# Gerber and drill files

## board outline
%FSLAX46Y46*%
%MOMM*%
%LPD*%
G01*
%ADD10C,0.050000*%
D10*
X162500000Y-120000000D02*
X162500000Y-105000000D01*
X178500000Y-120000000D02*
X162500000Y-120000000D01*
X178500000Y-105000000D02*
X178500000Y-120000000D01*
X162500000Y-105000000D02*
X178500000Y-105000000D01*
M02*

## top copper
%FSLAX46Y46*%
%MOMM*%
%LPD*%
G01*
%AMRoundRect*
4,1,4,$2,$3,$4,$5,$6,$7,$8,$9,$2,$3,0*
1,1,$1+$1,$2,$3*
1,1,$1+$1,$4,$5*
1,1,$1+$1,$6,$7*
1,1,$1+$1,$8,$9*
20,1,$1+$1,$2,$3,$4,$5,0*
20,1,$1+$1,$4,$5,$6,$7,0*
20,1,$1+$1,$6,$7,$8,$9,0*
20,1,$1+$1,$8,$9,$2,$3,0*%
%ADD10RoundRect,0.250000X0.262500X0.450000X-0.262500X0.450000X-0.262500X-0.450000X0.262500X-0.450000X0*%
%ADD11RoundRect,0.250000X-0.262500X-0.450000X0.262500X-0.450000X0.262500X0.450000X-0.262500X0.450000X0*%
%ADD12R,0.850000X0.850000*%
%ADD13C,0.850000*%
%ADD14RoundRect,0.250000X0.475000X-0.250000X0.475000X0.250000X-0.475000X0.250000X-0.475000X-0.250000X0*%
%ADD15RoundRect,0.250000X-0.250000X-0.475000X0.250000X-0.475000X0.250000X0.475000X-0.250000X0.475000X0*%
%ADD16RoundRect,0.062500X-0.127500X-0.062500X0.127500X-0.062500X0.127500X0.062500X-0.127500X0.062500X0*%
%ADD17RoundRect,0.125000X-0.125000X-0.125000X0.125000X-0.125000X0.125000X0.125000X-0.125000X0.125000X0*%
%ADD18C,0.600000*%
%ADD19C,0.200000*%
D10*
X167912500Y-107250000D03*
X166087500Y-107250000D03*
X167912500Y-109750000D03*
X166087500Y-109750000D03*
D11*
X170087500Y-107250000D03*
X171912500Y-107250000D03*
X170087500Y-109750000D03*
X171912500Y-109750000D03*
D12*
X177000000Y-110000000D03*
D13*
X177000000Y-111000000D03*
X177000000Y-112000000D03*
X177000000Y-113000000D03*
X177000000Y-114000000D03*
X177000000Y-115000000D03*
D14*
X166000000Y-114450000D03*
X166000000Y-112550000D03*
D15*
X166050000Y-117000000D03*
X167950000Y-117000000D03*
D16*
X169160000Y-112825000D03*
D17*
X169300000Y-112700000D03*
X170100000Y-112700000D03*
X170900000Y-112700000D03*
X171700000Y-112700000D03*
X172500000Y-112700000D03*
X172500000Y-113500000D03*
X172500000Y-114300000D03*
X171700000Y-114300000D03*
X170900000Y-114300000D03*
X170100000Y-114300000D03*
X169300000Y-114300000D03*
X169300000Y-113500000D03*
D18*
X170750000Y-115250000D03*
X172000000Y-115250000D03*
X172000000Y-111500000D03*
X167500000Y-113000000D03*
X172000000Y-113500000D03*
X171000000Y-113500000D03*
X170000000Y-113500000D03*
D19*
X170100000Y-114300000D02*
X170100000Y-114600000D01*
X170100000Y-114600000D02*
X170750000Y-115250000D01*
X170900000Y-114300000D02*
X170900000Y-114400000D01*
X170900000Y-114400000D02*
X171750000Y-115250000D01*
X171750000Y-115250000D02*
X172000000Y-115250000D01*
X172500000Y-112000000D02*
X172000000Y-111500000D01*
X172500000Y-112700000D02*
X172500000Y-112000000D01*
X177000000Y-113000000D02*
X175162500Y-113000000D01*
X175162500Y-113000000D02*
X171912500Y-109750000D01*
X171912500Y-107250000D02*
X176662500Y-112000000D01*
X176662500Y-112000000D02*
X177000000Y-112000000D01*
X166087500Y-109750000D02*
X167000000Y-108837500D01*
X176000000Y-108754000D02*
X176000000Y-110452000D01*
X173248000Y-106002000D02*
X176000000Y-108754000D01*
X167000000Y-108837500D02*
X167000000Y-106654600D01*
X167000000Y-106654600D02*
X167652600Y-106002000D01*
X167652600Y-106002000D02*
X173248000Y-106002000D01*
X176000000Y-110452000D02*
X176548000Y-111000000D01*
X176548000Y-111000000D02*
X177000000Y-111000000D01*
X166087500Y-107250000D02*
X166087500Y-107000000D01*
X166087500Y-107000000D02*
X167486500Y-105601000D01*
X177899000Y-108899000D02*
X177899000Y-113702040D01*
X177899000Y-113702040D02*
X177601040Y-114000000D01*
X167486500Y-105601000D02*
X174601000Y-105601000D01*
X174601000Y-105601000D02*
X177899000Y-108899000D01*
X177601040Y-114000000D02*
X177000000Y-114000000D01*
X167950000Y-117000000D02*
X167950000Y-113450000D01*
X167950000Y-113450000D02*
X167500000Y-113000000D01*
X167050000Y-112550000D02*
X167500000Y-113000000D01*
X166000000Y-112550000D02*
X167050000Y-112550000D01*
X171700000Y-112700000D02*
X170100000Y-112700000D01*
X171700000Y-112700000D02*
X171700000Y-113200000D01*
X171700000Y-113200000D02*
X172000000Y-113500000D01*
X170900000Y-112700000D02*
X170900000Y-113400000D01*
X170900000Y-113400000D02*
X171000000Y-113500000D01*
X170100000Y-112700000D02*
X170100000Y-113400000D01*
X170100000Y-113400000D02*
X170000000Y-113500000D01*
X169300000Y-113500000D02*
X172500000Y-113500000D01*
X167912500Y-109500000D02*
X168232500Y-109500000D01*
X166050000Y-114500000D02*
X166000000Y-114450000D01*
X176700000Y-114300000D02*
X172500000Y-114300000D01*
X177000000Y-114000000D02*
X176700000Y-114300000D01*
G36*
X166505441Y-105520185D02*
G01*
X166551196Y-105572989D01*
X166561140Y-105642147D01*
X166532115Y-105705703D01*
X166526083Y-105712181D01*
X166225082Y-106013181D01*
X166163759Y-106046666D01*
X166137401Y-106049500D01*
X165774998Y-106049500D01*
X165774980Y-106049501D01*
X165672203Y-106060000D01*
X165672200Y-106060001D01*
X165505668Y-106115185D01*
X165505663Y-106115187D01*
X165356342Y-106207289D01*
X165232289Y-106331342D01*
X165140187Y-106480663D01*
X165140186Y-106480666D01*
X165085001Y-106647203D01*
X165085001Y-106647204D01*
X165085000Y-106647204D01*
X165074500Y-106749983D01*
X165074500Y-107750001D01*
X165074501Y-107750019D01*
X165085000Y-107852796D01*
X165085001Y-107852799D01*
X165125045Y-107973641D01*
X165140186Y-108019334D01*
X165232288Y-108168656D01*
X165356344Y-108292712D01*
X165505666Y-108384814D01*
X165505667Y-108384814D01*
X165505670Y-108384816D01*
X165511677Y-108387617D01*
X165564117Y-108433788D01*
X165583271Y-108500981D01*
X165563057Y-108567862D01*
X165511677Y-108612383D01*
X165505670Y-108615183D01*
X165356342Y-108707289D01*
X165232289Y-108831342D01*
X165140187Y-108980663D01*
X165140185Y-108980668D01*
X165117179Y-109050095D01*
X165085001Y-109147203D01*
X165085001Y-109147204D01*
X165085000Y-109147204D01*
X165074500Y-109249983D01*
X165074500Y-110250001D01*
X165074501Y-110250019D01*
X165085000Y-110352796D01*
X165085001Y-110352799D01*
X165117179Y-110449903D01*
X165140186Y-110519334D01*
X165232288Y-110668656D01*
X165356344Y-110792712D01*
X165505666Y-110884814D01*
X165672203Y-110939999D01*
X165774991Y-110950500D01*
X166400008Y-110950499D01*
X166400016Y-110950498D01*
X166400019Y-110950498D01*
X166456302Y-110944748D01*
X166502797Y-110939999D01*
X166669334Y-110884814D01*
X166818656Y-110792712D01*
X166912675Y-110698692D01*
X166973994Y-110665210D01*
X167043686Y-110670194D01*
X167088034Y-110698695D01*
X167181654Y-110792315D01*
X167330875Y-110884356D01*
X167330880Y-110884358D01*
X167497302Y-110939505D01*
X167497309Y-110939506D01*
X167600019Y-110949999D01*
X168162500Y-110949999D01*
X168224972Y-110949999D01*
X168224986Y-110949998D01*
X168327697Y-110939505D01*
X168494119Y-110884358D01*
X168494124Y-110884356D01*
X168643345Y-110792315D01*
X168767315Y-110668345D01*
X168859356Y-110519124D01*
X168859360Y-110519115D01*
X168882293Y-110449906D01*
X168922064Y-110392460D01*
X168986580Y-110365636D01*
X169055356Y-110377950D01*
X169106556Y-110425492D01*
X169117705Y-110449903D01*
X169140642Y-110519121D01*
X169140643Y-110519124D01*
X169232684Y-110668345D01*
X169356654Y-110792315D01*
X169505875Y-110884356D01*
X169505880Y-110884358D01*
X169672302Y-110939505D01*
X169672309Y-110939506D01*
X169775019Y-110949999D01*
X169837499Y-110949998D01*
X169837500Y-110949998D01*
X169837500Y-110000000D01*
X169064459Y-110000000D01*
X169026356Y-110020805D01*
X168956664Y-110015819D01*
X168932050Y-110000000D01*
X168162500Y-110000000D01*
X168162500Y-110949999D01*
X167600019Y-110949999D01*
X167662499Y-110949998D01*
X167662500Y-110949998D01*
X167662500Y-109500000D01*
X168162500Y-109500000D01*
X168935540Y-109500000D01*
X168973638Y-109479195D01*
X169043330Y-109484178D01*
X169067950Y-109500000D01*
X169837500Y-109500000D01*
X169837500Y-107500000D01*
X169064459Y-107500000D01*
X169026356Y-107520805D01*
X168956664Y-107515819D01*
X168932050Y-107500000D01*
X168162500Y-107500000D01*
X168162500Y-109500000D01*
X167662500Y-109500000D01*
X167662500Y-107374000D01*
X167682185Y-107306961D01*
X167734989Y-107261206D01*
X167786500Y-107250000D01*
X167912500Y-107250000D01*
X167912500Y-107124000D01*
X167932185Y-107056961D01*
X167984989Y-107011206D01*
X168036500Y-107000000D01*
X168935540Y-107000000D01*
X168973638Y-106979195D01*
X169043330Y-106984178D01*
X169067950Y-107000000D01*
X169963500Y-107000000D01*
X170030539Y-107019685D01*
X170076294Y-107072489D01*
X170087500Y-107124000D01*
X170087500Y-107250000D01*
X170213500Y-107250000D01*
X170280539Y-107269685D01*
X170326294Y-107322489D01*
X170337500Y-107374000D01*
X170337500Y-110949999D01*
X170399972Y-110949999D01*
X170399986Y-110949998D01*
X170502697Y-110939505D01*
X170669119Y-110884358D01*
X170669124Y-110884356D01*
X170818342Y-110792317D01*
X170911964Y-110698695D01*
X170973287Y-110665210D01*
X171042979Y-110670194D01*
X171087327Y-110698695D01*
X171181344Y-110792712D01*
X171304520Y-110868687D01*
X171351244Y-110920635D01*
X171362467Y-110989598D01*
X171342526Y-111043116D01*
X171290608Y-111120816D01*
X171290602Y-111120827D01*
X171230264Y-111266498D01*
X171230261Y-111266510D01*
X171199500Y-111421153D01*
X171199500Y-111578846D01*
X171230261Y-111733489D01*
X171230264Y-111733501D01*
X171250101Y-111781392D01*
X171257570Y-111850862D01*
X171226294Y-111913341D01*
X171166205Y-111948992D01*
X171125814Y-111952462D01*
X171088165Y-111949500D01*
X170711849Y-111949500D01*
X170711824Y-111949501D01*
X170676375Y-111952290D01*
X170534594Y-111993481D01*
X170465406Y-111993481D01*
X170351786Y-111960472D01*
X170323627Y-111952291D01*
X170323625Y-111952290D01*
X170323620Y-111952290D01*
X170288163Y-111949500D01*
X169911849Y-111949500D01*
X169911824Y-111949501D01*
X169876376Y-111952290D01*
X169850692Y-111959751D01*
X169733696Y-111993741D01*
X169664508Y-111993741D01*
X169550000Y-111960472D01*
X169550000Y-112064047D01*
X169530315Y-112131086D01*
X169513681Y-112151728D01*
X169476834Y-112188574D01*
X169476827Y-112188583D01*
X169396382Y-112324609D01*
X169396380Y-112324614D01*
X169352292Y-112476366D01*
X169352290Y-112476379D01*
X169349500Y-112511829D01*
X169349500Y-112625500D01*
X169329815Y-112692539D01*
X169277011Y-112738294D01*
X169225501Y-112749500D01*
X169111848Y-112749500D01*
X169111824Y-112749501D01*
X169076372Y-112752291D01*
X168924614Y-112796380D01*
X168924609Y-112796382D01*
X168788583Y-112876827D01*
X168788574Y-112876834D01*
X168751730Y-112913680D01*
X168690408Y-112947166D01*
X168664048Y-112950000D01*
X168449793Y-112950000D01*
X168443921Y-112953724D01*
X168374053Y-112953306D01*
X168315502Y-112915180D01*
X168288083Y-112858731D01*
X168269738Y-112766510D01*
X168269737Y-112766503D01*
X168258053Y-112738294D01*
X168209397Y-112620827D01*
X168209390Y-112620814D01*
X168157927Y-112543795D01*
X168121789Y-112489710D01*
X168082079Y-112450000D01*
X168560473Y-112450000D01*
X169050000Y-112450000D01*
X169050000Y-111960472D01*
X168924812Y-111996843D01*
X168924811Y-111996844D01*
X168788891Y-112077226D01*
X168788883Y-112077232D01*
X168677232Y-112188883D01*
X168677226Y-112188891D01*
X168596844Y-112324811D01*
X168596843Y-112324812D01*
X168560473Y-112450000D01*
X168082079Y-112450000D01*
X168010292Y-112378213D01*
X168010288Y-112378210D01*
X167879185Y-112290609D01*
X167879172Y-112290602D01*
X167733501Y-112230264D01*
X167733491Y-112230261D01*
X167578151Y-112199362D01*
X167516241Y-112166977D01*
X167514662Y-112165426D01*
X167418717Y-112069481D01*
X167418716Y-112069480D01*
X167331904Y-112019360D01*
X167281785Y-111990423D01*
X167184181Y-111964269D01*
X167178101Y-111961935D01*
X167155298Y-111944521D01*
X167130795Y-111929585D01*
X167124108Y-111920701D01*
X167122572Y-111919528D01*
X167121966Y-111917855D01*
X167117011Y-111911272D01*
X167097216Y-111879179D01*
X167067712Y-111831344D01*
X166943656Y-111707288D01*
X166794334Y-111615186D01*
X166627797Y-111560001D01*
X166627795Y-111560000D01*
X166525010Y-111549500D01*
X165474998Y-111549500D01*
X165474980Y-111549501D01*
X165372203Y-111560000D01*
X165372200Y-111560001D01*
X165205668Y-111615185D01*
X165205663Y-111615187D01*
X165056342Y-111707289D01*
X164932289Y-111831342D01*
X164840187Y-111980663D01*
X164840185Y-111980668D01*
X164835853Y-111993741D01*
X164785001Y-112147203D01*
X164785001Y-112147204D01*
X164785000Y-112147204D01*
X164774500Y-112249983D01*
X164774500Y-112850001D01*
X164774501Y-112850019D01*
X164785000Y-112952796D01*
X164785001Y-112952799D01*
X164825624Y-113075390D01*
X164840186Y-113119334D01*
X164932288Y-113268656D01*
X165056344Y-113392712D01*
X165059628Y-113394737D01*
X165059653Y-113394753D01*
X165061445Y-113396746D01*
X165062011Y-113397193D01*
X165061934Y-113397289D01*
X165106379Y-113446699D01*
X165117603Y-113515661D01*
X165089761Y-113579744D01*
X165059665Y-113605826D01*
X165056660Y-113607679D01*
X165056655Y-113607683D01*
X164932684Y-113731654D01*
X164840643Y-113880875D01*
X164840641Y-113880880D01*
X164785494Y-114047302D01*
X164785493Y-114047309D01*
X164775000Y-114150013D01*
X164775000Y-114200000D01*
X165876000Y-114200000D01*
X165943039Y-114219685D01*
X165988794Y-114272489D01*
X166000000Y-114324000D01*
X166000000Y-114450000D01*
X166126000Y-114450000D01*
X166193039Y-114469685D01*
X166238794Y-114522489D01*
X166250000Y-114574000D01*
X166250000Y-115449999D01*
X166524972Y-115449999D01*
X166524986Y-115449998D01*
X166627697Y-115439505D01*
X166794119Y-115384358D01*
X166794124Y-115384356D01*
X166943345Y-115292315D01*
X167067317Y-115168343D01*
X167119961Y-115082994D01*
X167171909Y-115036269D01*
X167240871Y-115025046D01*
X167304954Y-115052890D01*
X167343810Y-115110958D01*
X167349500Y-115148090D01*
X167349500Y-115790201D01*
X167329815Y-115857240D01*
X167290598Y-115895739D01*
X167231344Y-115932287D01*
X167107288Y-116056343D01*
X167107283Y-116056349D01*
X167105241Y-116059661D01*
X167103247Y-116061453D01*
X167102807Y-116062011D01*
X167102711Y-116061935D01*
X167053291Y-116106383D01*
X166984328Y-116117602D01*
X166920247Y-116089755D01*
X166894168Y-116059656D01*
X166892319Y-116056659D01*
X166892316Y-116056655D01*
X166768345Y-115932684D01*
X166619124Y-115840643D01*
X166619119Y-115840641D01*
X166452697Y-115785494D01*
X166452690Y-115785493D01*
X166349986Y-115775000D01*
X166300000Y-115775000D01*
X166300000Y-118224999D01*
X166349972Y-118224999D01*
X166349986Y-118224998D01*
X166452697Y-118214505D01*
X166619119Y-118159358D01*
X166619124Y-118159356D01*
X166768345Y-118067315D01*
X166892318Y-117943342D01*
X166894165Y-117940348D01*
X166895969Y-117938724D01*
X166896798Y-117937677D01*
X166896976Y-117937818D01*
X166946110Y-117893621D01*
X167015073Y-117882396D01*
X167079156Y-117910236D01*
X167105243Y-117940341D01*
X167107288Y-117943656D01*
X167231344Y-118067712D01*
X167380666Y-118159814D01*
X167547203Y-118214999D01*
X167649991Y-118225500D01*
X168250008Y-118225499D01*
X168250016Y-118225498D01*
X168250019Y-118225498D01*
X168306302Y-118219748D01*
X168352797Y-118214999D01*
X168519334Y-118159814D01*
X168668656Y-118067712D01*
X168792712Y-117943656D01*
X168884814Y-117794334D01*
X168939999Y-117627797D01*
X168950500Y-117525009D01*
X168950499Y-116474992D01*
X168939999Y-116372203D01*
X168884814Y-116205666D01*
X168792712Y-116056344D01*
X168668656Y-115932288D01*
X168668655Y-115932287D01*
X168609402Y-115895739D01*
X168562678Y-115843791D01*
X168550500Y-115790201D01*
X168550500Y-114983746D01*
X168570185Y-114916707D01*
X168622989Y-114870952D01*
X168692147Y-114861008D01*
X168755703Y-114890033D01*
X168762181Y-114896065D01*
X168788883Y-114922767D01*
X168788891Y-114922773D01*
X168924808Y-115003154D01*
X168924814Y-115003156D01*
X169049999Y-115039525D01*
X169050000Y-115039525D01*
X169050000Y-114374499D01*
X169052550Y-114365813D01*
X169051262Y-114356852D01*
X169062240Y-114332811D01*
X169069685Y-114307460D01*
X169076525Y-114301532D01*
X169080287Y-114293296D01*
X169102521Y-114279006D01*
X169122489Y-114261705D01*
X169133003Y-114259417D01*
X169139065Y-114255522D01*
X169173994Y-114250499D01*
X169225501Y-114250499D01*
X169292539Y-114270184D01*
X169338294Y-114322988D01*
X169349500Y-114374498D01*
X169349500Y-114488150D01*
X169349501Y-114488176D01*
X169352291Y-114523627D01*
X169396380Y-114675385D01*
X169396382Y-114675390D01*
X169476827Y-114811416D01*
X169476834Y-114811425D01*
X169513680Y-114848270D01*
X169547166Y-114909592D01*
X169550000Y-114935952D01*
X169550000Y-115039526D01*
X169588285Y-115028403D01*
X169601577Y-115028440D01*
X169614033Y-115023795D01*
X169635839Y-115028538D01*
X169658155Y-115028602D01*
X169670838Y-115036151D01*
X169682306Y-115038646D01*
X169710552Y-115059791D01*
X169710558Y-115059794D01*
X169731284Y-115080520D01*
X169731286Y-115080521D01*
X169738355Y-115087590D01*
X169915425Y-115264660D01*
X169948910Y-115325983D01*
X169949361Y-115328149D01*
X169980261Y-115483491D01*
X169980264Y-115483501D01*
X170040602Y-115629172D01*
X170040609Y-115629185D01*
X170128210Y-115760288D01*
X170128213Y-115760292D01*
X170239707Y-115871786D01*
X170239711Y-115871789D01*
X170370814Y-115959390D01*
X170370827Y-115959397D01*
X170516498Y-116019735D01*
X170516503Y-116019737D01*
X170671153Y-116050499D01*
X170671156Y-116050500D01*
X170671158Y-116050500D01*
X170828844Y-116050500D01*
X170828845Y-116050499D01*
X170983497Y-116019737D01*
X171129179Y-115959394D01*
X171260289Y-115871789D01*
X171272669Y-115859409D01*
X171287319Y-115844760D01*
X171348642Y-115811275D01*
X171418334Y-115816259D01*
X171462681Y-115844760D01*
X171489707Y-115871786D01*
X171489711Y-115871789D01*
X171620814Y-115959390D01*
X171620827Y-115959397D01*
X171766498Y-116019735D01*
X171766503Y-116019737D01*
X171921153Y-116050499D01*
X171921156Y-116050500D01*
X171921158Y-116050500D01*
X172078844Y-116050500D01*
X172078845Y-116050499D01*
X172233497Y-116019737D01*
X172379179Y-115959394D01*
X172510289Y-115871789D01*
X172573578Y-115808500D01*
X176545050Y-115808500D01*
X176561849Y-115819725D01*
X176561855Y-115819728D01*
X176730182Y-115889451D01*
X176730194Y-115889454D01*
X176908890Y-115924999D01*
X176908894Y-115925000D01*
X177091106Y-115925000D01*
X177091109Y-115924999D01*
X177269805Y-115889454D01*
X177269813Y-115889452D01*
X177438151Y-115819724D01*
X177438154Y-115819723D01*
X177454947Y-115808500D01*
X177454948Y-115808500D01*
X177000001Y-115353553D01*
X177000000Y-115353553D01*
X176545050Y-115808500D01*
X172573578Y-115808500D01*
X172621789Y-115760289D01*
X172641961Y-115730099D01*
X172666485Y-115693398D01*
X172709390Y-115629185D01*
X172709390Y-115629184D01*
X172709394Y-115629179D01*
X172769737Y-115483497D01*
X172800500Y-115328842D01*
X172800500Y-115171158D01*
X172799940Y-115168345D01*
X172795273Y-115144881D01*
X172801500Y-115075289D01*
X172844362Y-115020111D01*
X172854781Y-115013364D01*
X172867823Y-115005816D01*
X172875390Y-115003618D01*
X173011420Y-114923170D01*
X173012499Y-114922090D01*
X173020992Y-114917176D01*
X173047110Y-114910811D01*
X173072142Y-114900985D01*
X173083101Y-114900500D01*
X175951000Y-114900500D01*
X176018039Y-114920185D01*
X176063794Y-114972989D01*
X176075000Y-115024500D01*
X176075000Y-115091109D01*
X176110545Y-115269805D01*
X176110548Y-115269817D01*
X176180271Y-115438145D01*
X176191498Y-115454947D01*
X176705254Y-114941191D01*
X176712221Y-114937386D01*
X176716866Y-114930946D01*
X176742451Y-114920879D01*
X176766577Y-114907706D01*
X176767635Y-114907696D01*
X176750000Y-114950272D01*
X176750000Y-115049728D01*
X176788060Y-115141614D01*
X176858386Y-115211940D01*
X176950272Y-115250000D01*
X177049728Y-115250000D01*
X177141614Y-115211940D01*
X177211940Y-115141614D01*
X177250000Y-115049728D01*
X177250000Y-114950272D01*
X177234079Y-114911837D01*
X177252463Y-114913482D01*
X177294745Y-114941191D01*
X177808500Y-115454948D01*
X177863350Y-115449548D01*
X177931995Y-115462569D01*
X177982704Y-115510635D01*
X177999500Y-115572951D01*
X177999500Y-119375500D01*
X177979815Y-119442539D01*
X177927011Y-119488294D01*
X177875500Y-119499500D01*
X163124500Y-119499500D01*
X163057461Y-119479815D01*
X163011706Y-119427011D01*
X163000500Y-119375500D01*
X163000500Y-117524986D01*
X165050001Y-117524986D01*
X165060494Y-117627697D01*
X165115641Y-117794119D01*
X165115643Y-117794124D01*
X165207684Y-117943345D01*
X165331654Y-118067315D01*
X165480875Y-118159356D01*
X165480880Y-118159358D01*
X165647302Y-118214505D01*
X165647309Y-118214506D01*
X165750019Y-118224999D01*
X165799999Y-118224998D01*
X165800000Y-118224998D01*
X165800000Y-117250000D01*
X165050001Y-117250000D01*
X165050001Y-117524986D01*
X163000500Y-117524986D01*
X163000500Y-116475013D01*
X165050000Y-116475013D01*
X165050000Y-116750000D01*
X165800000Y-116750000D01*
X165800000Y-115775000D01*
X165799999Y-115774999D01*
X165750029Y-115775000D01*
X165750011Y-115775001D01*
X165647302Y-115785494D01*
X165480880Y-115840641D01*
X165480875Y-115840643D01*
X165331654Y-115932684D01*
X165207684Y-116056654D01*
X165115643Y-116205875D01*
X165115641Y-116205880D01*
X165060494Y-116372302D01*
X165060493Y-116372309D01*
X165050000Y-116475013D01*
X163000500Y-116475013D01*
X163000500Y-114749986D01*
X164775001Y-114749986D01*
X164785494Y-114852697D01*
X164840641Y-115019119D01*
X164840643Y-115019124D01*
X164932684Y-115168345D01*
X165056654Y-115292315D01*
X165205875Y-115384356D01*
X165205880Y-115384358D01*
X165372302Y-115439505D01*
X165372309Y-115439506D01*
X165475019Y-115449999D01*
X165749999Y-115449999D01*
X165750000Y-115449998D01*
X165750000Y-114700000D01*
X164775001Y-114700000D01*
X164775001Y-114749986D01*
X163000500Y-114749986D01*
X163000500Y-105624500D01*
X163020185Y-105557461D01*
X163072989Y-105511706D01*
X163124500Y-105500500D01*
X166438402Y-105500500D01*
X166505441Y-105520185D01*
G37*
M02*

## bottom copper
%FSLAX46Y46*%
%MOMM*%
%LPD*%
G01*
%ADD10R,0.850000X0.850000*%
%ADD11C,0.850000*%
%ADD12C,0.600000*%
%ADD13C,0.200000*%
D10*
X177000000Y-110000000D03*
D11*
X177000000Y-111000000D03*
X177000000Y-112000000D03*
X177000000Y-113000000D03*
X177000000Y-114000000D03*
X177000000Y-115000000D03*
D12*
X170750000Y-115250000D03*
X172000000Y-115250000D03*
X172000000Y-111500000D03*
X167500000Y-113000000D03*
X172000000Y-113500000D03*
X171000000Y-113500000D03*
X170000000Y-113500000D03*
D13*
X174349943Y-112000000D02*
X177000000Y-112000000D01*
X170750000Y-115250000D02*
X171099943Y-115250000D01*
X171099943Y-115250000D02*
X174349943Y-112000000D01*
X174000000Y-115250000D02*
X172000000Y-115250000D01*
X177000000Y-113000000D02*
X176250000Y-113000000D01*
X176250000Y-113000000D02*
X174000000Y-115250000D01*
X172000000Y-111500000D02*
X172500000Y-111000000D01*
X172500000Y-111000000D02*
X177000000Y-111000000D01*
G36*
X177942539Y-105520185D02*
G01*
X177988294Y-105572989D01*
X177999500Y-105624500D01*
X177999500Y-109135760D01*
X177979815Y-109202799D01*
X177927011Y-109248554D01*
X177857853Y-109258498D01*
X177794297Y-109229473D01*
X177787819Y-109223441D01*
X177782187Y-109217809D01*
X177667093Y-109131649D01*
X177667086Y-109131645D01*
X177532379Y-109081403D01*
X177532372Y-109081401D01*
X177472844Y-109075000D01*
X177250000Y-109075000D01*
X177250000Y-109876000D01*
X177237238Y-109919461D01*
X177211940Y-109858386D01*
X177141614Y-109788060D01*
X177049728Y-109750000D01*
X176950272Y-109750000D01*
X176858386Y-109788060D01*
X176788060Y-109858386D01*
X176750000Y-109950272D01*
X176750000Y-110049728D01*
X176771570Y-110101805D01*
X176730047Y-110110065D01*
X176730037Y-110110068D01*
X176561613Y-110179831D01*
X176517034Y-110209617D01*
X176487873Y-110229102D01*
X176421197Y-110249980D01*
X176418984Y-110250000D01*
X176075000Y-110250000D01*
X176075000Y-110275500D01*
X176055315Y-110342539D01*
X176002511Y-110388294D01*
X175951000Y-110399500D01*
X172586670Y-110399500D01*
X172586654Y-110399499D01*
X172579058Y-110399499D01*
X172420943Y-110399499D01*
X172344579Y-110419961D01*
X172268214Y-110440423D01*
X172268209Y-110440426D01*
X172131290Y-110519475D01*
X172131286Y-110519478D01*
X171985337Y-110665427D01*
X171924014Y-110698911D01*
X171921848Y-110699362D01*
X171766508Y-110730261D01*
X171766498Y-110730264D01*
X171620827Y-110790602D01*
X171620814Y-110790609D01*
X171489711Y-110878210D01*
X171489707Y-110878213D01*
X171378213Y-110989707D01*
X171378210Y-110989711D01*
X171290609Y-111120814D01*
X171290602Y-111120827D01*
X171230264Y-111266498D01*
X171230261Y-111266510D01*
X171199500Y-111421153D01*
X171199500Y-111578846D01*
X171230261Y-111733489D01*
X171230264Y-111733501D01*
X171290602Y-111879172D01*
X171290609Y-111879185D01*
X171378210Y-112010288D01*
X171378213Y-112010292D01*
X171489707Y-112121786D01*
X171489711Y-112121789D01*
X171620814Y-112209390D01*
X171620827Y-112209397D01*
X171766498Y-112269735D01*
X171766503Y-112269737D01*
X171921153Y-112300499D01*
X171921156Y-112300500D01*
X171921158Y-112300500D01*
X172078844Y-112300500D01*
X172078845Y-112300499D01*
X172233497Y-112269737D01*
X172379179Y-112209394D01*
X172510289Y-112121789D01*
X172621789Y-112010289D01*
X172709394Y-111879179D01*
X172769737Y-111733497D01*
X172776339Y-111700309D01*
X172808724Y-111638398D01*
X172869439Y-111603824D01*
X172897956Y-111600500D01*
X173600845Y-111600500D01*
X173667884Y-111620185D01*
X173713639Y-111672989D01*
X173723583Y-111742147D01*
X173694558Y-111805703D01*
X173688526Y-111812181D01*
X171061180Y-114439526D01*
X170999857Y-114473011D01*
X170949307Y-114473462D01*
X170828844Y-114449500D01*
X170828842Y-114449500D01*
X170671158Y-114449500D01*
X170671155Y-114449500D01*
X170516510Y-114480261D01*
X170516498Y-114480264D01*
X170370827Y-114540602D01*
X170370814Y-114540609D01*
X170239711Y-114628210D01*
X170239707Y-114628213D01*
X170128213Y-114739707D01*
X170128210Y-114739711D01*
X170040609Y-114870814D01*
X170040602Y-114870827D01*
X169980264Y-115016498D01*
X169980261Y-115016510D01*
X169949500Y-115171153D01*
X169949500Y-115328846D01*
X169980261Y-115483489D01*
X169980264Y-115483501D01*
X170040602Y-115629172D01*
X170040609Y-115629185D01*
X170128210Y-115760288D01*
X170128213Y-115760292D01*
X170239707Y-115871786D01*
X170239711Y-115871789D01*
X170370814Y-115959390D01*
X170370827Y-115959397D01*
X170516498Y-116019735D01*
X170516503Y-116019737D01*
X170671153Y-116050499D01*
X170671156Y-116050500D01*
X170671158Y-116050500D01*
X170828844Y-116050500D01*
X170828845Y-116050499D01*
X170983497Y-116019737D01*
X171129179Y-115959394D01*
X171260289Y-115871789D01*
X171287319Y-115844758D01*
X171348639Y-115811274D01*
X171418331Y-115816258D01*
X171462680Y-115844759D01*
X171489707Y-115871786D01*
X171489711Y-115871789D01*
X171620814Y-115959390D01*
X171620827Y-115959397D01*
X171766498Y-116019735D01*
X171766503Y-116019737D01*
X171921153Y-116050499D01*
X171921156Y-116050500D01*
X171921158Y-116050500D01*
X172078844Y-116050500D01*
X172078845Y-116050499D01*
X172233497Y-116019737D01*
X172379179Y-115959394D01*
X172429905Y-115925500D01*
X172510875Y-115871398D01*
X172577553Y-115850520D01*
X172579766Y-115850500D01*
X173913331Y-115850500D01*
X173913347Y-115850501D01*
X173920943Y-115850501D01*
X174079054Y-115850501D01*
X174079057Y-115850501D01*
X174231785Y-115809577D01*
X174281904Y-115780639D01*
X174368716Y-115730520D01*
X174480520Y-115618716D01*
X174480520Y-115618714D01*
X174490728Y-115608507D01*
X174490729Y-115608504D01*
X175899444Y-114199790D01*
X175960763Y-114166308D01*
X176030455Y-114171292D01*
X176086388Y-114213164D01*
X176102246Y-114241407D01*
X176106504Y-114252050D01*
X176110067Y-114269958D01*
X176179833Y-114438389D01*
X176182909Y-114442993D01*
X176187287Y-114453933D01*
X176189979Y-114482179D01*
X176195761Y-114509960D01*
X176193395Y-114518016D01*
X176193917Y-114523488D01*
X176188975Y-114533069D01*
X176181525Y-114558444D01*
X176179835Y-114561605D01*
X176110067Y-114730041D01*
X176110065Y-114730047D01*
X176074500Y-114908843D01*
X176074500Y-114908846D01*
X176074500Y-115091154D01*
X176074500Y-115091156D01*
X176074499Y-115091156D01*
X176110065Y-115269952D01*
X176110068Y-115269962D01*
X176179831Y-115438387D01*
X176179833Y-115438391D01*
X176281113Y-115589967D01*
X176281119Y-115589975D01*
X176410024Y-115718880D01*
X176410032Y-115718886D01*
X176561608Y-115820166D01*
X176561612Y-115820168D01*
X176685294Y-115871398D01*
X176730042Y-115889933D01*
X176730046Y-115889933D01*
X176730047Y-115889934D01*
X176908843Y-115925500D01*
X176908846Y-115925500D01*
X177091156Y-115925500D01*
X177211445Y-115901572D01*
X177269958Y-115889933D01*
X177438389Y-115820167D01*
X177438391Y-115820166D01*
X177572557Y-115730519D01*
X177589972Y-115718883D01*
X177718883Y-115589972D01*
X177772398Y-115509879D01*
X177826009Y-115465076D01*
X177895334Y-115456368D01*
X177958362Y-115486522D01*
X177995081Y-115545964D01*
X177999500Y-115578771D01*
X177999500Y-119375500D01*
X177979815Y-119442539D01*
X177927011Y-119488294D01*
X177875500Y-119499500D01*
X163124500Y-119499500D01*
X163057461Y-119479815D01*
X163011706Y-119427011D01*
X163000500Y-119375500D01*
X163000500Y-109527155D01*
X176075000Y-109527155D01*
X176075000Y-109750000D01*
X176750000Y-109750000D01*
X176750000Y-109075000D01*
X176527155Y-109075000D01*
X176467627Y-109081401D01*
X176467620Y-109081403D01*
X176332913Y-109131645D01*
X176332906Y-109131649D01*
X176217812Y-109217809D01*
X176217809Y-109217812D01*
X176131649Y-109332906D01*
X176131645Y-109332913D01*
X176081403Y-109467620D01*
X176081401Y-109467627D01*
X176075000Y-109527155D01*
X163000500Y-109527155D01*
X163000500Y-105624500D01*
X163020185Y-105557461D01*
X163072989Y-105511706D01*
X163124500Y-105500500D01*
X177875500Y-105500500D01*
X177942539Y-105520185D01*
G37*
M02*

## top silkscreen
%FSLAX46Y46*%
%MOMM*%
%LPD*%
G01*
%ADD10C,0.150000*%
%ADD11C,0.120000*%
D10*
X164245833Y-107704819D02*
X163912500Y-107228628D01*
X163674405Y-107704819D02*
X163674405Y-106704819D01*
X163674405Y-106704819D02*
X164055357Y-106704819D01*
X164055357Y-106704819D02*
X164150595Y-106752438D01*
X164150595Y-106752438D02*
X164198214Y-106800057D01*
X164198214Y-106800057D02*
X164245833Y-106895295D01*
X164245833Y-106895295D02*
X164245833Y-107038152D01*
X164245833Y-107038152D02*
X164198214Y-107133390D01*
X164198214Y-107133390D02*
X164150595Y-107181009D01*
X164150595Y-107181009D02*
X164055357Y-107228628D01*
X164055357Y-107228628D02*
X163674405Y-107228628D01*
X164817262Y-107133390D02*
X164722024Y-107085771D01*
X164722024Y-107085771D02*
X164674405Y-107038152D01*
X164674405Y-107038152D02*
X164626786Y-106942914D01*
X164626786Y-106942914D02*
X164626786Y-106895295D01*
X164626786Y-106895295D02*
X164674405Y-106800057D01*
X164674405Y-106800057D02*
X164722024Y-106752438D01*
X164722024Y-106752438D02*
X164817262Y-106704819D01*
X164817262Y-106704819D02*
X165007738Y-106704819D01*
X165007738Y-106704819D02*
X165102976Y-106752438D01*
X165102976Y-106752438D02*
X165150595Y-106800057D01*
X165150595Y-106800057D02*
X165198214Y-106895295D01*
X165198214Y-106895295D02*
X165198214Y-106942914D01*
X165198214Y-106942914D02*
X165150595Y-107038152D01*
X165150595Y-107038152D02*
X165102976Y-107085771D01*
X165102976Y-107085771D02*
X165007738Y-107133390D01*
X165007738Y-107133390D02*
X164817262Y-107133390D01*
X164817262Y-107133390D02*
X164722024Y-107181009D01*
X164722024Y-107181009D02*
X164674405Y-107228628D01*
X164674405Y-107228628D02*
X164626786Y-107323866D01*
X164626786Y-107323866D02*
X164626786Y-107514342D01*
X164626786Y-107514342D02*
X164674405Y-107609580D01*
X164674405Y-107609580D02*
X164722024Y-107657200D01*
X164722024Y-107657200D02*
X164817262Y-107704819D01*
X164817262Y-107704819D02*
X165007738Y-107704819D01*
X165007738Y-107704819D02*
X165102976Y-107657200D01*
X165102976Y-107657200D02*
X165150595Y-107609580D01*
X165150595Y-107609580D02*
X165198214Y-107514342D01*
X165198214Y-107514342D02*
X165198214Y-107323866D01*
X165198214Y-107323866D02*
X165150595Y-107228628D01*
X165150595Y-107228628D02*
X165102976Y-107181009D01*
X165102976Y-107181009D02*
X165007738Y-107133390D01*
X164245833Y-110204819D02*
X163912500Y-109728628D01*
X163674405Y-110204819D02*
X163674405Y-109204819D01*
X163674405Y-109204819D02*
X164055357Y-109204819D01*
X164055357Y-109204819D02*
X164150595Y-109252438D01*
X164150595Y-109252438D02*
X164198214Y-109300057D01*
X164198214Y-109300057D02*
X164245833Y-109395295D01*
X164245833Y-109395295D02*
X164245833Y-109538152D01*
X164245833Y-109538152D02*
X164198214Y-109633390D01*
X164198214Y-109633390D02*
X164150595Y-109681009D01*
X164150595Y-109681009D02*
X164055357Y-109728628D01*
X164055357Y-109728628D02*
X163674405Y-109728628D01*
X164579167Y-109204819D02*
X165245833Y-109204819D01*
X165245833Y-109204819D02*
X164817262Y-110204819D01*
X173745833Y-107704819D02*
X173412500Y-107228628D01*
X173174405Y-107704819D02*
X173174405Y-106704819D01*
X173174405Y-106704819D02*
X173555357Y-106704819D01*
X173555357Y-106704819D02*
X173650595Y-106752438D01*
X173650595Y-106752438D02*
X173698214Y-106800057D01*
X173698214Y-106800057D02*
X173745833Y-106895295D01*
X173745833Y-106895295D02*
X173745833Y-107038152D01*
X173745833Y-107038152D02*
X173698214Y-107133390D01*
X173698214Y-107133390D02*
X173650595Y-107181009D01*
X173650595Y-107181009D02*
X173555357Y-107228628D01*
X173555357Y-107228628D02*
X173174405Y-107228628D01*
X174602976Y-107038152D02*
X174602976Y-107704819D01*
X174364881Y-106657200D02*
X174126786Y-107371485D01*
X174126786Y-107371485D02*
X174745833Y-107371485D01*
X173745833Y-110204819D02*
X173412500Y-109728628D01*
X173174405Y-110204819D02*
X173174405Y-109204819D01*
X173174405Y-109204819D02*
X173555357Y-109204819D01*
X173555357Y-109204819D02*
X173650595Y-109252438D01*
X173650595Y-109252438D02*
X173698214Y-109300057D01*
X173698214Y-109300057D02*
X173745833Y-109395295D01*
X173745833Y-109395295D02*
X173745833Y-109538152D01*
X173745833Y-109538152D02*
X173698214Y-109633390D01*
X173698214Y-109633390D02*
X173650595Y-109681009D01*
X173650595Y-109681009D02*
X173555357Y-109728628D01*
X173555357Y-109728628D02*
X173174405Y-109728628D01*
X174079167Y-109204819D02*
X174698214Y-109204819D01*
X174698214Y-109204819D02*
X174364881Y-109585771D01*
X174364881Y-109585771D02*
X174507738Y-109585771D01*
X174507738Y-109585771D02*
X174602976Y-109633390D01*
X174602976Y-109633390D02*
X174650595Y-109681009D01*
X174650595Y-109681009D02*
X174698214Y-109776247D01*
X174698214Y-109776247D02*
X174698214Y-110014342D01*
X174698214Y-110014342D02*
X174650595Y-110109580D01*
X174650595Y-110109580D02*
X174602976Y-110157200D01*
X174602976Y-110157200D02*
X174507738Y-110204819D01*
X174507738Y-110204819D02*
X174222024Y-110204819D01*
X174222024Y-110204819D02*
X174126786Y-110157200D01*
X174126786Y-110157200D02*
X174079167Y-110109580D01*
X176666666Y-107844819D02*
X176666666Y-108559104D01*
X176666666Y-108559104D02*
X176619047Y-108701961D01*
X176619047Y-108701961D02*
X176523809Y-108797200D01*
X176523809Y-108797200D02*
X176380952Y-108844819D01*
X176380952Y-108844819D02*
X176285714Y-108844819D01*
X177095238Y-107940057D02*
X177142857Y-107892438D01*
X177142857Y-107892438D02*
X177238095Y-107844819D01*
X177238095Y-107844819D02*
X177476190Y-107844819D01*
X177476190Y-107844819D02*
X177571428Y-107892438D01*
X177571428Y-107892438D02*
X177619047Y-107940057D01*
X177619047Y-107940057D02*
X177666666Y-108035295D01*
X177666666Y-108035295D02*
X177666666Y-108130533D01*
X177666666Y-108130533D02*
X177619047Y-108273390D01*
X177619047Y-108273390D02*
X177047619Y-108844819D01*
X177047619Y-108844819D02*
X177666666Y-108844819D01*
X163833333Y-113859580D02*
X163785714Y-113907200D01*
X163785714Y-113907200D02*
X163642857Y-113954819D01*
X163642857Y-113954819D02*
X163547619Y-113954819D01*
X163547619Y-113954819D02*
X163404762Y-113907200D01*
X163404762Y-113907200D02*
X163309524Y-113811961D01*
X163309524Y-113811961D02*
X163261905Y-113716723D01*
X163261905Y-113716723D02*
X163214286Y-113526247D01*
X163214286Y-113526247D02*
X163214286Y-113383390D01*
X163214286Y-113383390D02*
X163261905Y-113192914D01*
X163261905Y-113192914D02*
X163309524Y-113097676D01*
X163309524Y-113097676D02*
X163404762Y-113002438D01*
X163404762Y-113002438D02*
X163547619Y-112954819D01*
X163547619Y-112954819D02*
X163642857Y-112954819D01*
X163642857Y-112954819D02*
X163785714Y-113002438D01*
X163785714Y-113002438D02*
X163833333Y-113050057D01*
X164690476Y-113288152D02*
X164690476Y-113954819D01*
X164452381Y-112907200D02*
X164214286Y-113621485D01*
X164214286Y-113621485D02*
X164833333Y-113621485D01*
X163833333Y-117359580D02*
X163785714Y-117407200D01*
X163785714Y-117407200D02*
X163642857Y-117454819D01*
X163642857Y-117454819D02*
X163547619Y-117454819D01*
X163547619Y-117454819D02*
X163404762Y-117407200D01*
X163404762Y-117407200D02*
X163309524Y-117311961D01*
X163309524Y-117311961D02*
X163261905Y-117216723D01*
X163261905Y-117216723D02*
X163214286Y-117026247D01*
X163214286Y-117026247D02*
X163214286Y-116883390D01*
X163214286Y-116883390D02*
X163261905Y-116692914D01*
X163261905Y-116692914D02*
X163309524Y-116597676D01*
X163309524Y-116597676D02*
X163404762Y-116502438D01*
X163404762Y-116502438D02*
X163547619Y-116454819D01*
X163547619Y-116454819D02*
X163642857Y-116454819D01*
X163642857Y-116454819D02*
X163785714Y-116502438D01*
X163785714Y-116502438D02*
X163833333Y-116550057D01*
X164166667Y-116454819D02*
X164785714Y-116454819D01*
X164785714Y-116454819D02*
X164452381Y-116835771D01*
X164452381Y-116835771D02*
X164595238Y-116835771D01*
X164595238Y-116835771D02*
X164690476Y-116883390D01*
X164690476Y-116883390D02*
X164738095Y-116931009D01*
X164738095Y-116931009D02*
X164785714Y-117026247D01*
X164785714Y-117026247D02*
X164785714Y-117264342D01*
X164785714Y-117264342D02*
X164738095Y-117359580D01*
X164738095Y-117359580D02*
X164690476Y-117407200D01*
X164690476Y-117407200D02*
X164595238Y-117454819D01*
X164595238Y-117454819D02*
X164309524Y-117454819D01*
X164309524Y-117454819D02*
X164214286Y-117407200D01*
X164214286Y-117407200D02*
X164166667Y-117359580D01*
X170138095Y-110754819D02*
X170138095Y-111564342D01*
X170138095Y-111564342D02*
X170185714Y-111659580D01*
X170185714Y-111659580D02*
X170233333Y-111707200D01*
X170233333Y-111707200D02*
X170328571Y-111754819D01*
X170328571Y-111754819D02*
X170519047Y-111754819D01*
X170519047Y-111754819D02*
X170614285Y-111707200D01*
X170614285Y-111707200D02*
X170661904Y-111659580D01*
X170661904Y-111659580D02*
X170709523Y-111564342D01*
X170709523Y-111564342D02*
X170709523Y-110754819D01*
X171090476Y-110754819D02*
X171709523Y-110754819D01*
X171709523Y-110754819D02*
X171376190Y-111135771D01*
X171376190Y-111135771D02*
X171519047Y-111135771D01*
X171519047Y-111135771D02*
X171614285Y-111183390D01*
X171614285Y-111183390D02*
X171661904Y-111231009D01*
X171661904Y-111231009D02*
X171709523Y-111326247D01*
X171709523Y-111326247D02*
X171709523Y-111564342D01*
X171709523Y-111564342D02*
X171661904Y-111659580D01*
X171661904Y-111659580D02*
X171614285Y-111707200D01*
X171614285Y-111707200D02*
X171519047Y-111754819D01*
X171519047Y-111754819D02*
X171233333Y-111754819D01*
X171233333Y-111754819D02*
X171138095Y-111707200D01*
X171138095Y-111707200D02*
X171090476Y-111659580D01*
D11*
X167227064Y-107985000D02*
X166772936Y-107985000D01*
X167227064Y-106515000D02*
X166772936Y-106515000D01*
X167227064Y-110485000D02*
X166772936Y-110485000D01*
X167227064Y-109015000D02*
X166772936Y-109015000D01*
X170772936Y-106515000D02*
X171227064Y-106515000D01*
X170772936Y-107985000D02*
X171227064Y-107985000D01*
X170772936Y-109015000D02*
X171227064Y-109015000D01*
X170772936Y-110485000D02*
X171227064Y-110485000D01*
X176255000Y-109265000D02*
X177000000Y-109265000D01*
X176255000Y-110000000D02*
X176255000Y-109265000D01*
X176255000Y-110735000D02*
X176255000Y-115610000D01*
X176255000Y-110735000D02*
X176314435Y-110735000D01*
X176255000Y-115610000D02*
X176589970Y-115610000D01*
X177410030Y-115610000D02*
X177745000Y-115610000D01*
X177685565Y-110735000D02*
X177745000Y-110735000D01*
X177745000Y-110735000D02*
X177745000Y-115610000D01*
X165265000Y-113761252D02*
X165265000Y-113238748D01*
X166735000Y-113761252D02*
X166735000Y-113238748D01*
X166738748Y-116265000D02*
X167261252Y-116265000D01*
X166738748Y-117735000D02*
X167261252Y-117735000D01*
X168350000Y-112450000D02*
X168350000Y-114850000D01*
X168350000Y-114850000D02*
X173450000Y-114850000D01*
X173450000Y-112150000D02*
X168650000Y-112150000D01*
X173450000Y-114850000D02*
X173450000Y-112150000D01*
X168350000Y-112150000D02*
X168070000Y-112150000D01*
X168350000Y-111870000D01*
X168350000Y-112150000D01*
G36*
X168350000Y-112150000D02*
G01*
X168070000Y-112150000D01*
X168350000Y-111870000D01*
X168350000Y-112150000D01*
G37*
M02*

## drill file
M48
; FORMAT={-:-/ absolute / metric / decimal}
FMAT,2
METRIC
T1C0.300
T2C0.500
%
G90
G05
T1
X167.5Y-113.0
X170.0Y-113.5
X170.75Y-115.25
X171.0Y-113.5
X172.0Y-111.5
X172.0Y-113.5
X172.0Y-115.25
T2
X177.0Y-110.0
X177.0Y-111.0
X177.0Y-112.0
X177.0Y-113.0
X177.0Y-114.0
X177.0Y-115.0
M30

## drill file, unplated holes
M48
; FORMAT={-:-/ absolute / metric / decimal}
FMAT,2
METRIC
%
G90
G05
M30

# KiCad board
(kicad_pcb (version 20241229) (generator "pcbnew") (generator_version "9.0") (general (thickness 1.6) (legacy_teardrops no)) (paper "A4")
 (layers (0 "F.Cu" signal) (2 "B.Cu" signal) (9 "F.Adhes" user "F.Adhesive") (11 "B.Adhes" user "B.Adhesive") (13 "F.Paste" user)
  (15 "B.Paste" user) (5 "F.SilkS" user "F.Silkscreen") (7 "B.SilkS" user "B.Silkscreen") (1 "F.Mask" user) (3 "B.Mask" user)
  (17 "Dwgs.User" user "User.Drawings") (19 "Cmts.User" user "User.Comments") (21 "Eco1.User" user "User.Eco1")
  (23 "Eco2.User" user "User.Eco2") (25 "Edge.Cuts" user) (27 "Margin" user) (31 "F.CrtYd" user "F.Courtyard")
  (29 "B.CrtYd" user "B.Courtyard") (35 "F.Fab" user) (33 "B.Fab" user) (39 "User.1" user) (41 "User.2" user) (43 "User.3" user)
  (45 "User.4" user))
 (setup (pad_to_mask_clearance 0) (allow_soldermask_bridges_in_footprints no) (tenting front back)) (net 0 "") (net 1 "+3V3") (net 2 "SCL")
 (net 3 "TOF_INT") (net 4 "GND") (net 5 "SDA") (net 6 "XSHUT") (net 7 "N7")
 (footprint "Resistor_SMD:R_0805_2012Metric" (layer "F.Cu") (at 171 107.25)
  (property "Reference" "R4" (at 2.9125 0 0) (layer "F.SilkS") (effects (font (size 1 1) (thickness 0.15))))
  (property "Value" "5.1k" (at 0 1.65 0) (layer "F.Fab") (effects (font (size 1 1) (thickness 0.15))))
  (fp_line (start -0.227064 -0.735) (end 0.227064 -0.735) (stroke (width 0.12) (type solid)) (layer "F.SilkS"))
  (fp_line (start -0.227064 0.735) (end 0.227064 0.735) (stroke (width 0.12) (type solid)) (layer "F.SilkS"))
  (pad "1" smd roundrect (at -0.9125 0) (size 1.025 1.4) (layers "F.Cu" "F.Mask" "F.Paste") (roundrect_rratio 0.243902) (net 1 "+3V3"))
  (pad "2" smd roundrect (at 0.9125 0) (size 1.025 1.4) (layers "F.Cu" "F.Mask" "F.Paste") (roundrect_rratio 0.243902) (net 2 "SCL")))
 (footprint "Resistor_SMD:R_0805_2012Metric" (layer "F.Cu") (at 167 107.25 180)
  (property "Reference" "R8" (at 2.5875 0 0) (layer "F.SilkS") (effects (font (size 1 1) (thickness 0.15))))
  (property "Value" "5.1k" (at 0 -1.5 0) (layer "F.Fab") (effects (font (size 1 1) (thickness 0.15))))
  (fp_line (start -0.227064 0.735) (end 0.227064 0.735) (stroke (width 0.12) (type solid)) (layer "F.SilkS"))
  (fp_line (start -0.227064 -0.735) (end 0.227064 -0.735) (stroke (width 0.12) (type solid)) (layer "F.SilkS"))
  (pad "1" smd roundrect (at -0.9125 0 180) (size 1.025 1.4) (layers "F.Cu" "F.Mask" "F.Paste") (roundrect_rratio 0.243902) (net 1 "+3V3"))
  (pad "2" smd roundrect (at 0.9125 0 180) (size 1.025 1.4) (layers "F.Cu" "F.Mask" "F.Paste") (roundrect_rratio 0.243902) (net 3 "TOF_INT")))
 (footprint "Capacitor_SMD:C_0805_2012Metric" (layer "F.Cu") (at 166 113.5 90)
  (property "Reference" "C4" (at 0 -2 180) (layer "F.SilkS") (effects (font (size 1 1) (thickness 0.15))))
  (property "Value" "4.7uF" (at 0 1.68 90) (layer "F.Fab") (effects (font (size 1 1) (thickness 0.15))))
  (fp_line (start -0.261252 -0.735) (end 0.261252 -0.735) (stroke (width 0.12) (type solid)) (layer "F.SilkS"))
  (fp_line (start -0.261252 0.735) (end 0.261252 0.735) (stroke (width 0.12) (type solid)) (layer "F.SilkS"))
  (pad "1" smd roundrect (at -0.95 0 90) (size 1 1.45) (layers "F.Cu" "F.Mask" "F.Paste") (roundrect_rratio 0.25) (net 1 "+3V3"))
  (pad "2" smd roundrect (at 0.95 0 90) (size 1 1.45) (layers "F.Cu" "F.Mask" "F.Paste") (roundrect_rratio 0.25) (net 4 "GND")))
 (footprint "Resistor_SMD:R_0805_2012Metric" (layer "F.Cu") (at 171 109.75)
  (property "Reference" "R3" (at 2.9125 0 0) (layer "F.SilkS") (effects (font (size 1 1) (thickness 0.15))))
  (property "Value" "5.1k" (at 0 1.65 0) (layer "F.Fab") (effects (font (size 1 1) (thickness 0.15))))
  (fp_line (start -0.227064 -0.735) (end 0.227064 -0.735) (stroke (width 0.12) (type solid)) (layer "F.SilkS"))
  (fp_line (start -0.227064 0.735) (end 0.227064 0.735) (stroke (width 0.12) (type solid)) (layer "F.SilkS"))
  (pad "1" smd roundrect (at -0.9125 0) (size 1.025 1.4) (layers "F.Cu" "F.Mask" "F.Paste") (roundrect_rratio 0.243902) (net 1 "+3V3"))
  (pad "2" smd roundrect (at 0.9125 0) (size 1.025 1.4) (layers "F.Cu" "F.Mask" "F.Paste") (roundrect_rratio 0.243902) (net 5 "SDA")))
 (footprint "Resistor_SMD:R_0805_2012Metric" (layer "F.Cu") (at 167 109.75 180)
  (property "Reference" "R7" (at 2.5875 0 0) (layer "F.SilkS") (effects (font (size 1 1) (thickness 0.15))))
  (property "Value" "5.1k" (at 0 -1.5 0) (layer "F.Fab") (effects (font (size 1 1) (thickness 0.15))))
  (fp_line (start -0.227064 0.735) (end 0.227064 0.735) (stroke (width 0.12) (type solid)) (layer "F.SilkS"))
  (fp_line (start -0.227064 -0.735) (end 0.227064 -0.735) (stroke (width 0.12) (type solid)) (layer "F.SilkS"))
  (pad "1" smd roundrect (at -0.9125 0 180) (size 1.025 1.4) (layers "F.Cu" "F.Mask" "F.Paste") (roundrect_rratio 0.243902) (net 1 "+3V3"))
  (pad "2" smd roundrect (at 0.9125 0 180) (size 1.025 1.4) (layers "F.Cu" "F.Mask" "F.Paste") (roundrect_rratio 0.243902) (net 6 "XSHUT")))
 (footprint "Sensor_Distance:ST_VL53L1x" (layer "F.Cu") (at 170.9 113.5)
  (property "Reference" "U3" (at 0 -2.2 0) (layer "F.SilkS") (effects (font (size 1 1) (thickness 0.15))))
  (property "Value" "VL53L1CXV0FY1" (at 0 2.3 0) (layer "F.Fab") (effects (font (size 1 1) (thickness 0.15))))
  (fp_line (start -2.55 -1.05) (end -2.55 1.35) (stroke (width 0.12) (type solid)) (layer "F.SilkS"))
  (fp_line (start -2.55 1.35) (end 2.55 1.35) (stroke (width 0.12) (type solid)) (layer "F.SilkS"))
  (fp_line (start 2.55 -1.35) (end -2.25 -1.35) (stroke (width 0.12) (type solid)) (layer "F.SilkS"))
  (fp_line (start 2.55 1.35) (end 2.55 -1.35) (stroke (width 0.12) (type solid)) (layer "F.SilkS"))
  (fp_poly
   (pts (xy -2.55 -1.35) (xy -2.83 -1.35) (xy -2.55 -1.63) (xy -2.55 -1.35)) (stroke (width 0.12) (type solid)) (fill yes) (layer "F.SilkS"))
  (pad "1" smd roundrect (at -1.74 -0.675) (size 0.38 0.25) (layers "F.Cu" "F.Mask" "F.Paste") (roundrect_rratio 0.25) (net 1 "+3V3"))
  (pad "1" smd roundrect (at -1.6 -0.8) (size 0.5 0.5) (layers "F.Cu" "F.Mask" "F.Paste") (roundrect_rratio 0.25) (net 1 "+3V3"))
  (pad "2" smd roundrect (at -0.8 -0.8) (size 0.5 0.5) (layers "F.Cu" "F.Mask" "F.Paste") (roundrect_rratio 0.25) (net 4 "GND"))
  (pad "3" smd roundrect (at 0 -0.8) (size 0.5 0.5) (layers "F.Cu" "F.Mask" "F.Paste") (roundrect_rratio 0.25) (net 4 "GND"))
  (pad "4" smd roundrect (at 0.8 -0.8) (size 0.5 0.5) (layers "F.Cu" "F.Mask" "F.Paste") (roundrect_rratio 0.25) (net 4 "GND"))
  (pad "5" smd roundrect (at 1.6 -0.8) (size 0.5 0.5) (layers "F.Cu" "F.Mask" "F.Paste") (roundrect_rratio 0.25) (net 6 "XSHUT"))
  (pad "6" smd roundrect (at 1.6 0) (size 0.5 0.5) (layers "F.Cu" "F.Mask" "F.Paste") (roundrect_rratio 0.25) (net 4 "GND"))
  (pad "7" smd roundrect (at 1.6 0.8) (size 0.5 0.5) (layers "F.Cu" "F.Mask" "F.Paste") (roundrect_rratio 0.25) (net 3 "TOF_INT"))
  (pad "8" smd roundrect (at 0.8 0.8) (size 0.5 0.5) (layers "F.Cu" "F.Mask" "F.Paste") (roundrect_rratio 0.25) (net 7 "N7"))
  (pad "9" smd roundrect (at 0 0.8) (size 0.5 0.5) (layers "F.Cu" "F.Mask" "F.Paste") (roundrect_rratio 0.25) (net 5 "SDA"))
  (pad "10" smd roundrect (at -0.8 0.8) (size 0.5 0.5) (layers "F.Cu" "F.Mask" "F.Paste") (roundrect_rratio 0.25) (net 2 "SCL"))
  (pad "11" smd roundrect (at -1.6 0.8) (size 0.5 0.5) (layers "F.Cu" "F.Mask" "F.Paste") (roundrect_rratio 0.25) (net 1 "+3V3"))
  (pad "12" smd roundrect (at -1.6 0) (size 0.5 0.5) (layers "F.Cu" "F.Mask" "F.Paste") (roundrect_rratio 0.25) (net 4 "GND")))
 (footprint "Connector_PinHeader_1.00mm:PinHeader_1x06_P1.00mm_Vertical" (layer "F.Cu") (at 177 110)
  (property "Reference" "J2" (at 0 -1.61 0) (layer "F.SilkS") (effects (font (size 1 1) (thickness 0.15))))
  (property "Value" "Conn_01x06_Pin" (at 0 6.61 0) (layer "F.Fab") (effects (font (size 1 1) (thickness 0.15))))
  (fp_line (start -0.745 -0.735) (end 0 -0.735) (stroke (width 0.12) (type solid)) (layer "F.SilkS"))
  (fp_line (start -0.745 0) (end -0.745 -0.735) (stroke (width 0.12) (type solid)) (layer "F.SilkS"))
  (fp_line (start -0.745 0.735) (end -0.745 5.61) (stroke (width 0.12) (type solid)) (layer "F.SilkS"))
  (fp_line (start -0.745 0.735) (end -0.685565 0.735) (stroke (width 0.12) (type solid)) (layer "F.SilkS"))
  (fp_line (start -0.745 5.61) (end -0.41003 5.61) (stroke (width 0.12) (type solid)) (layer "F.SilkS"))
  (fp_line (start 0.41003 5.61) (end 0.745 5.61) (stroke (width 0.12) (type solid)) (layer "F.SilkS"))
  (fp_line (start 0.685565 0.735) (end 0.745 0.735) (stroke (width 0.12) (type solid)) (layer "F.SilkS"))
  (fp_line (start 0.745 0.735) (end 0.745 5.61) (stroke (width 0.12) (type solid)) (layer "F.SilkS"))
  (pad "1" thru_hole rect (at 0 0) (size 0.85 0.85) (drill 0.5) (layers "*.Cu" "*.Mask") (remove_unused_layers no) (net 4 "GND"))
  (pad "2" thru_hole circle (at 0 1) (size 0.85 0.85) (drill 0.5) (layers "*.Cu" "*.Mask") (remove_unused_layers no) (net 6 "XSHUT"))
  (pad "3" thru_hole circle (at 0 2) (size 0.85 0.85) (drill 0.5) (layers "*.Cu" "*.Mask") (remove_unused_layers no) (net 2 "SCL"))
  (pad "4" thru_hole circle (at 0 3) (size 0.85 0.85) (drill 0.5) (layers "*.Cu" "*.Mask") (remove_unused_layers no) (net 5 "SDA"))
  (pad "5" thru_hole circle (at 0 4) (size 0.85 0.85) (drill 0.5) (layers "*.Cu" "*.Mask") (remove_unused_layers no) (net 3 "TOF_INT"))
  (pad "6" thru_hole circle (at 0 5) (size 0.85 0.85) (drill 0.5) (layers "*.Cu" "*.Mask") (remove_unused_layers no) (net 1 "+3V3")))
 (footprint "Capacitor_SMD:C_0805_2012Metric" (layer "F.Cu") (at 167 117)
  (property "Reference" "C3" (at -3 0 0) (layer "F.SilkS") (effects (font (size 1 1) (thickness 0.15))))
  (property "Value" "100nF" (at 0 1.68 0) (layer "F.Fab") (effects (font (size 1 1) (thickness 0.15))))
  (fp_line (start -0.261252 -0.735) (end 0.261252 -0.735) (stroke (width 0.12) (type solid)) (layer "F.SilkS"))
  (fp_line (start -0.261252 0.735) (end 0.261252 0.735) (stroke (width 0.12) (type solid)) (layer "F.SilkS"))
  (pad "1" smd roundrect (at -0.95 0) (size 1 1.45) (layers "F.Cu" "F.Mask" "F.Paste") (roundrect_rratio 0.25) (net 1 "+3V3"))
  (pad "2" smd roundrect (at 0.95 0) (size 1 1.45) (layers "F.Cu" "F.Mask" "F.Paste") (roundrect_rratio 0.25) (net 4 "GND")))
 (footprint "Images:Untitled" (layer "B.Cu") (at 167.5 110 180)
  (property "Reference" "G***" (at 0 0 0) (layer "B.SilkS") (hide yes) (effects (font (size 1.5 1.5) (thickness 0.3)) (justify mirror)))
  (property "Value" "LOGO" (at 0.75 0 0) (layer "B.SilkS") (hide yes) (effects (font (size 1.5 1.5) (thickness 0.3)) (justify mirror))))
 (gr_line (start 178.5 120) (end 162.5 120) (stroke (width 0.05) (type default)) (layer "Edge.Cuts"))
 (gr_line (start 162.5 120) (end 162.5 105) (stroke (width 0.05) (type default)) (layer "Edge.Cuts"))
 (gr_line (start 162.5 105) (end 178.5 105) (stroke (width 0.05) (type default)) (layer "Edge.Cuts"))
 (gr_line (start 178.5 105) (end 178.5 120) (stroke (width 0.05) (type default)) (layer "Edge.Cuts"))
 (segment (start 170.1 113.4) (end 170 113.5) (width 0.2) (layer "F.Cu") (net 4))
 (segment (start 171.7 113.2) (end 172 113.5) (width 0.2) (layer "F.Cu") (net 4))
 (segment (start 169.3 113.5) (end 172.5 113.5) (width 0.2) (layer "F.Cu") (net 4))
 (segment (start 167.95 117) (end 167.95 113.45) (width 0.2) (layer "F.Cu") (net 4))
 (segment (start 166 112.55) (end 167.05 112.55) (width 0.2) (layer "F.Cu") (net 4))
 (segment (start 167.95 113.45) (end 167.5 113) (width 0.2) (layer "F.Cu") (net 4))
 (segment (start 167.05 112.55) (end 167.5 113) (width 0.2) (layer "F.Cu") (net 4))
 (segment (start 170.1 112.7) (end 170.1 113.4) (width 0.2) (layer "F.Cu") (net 4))
 (segment (start 171.7 112.7) (end 170.1 112.7) (width 0.2) (layer "F.Cu") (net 4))
 (segment (start 171.7 112.7) (end 171.7 113.2) (width 0.2) (layer "F.Cu") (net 4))
 (segment (start 170.9 113.4) (end 171 113.5) (width 0.2) (layer "F.Cu") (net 4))
 (segment (start 170.9 112.7) (end 170.9 113.4) (width 0.2) (layer "F.Cu") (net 4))
 (via (at 171 113.5) (size 0.6) (drill 0.3) (layers "F.Cu" "B.Cu") (free yes) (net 4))
 (via (at 172 113.5) (size 0.6) (drill 0.3) (layers "F.Cu" "B.Cu") (free yes) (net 4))
 (via (at 170 113.5) (size 0.6) (drill 0.3) (layers "F.Cu" "B.Cu") (free yes) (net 4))
 (via (at 167.5 113) (size 0.6) (drill 0.3) (layers "F.Cu" "B.Cu") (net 4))
 (segment (start 166.05 114.5) (end 166 114.45) (width 0.2) (layer "F.Cu") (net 1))
 (segment (start 167.9125 109.5) (end 168.2325 109.5) (width 0.2) (layer "F.Cu") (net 1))
 (segment (start 175.1625 113) (end 171.9125 109.75) (width 0.2) (layer "F.Cu") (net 5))
 (segment (start 177 113) (end 175.1625 113) (width 0.2) (layer "F.Cu") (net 5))
 (segment (start 171.75 115.25) (end 172 115.25) (width 0.2) (layer "F.Cu") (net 5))
 (segment (start 170.9 114.4) (end 171.75 115.25) (width 0.2) (layer "F.Cu") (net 5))
 (segment (start 170.9 114.3) (end 170.9 114.4) (width 0.2) (layer "F.Cu") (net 5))
 (via (at 172 115.25) (size 0.6) (drill 0.3) (layers "F.Cu" "B.Cu") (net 5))
 (segment (start 177 113) (end 176.25 113) (width 0.2) (layer "B.Cu") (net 5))
 (segment (start 174 115.25) (end 172 115.25) (width 0.2) (layer "B.Cu") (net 5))
 (segment (start 176.25 113) (end 174 115.25) (width 0.2) (layer "B.Cu") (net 5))
 (segment (start 176.6625 112) (end 177 112) (width 0.2) (layer "F.Cu") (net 2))
 (segment (start 171.9125 107.25) (end 176.6625 112) (width 0.2) (layer "F.Cu") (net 2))
 (segment (start 170.1 114.6) (end 170.75 115.25) (width 0.2) (layer "F.Cu") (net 2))
 (segment (start 170.1 114.3) (end 170.1 114.6) (width 0.2) (layer "F.Cu") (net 2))
 (via (at 170.75 115.25) (size 0.6) (drill 0.3) (layers "F.Cu" "B.Cu") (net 2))
 (segment (start 174.349943 112) (end 177 112) (width 0.2) (layer "B.Cu") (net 2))
 (segment (start 171.099943 115.25) (end 174.349943 112) (width 0.2) (layer "B.Cu") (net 2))
 (segment (start 170.75 115.25) (end 171.099943 115.25) (width 0.2) (layer "B.Cu") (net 2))
 (segment (start 176 110.452) (end 176.548 111) (width 0.2) (layer "F.Cu") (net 6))
 (segment (start 176.548 111) (end 177 111) (width 0.2) (layer "F.Cu") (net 6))
 (segment (start 173.248 106.002) (end 176 108.754) (width 0.2) (layer "F.Cu") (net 6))
 (segment (start 167.6526 106.002) (end 173.248 106.002) (width 0.2) (layer "F.Cu") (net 6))
 (segment (start 167 108.8375) (end 167 106.6546) (width 0.2) (layer "F.Cu") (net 6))
 (segment (start 166.0875 109.75) (end 167 108.8375) (width 0.2) (layer "F.Cu") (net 6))
 (segment (start 172.5 112) (end 172 111.5) (width 0.2) (layer "F.Cu") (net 6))
 (segment (start 167 106.6546) (end 167.6526 106.002) (width 0.2) (layer "F.Cu") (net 6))
 (segment (start 176 108.754) (end 176 110.452) (width 0.2) (layer "F.Cu") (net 6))
 (segment (start 172.5 112.7) (end 172.5 112) (width 0.2) (layer "F.Cu") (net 6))
 (via (at 172 111.5) (size 0.6) (drill 0.3) (layers "F.Cu" "B.Cu") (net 6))
 (segment (start 172 111.5) (end 172.5 111) (width 0.2) (layer "B.Cu") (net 6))
 (segment (start 172.5 111) (end 177 111) (width 0.2) (layer "B.Cu") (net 6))
 (segment (start 174.601 105.601) (end 177.899 108.899) (width 0.2) (layer "F.Cu") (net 3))
 (segment (start 177.899 113.70204) (end 177.60104 114) (width 0.2) (layer "F.Cu") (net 3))
 (segment (start 177 114) (end 176.7 114.3) (width 0.2) (layer "F.Cu") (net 3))
 (segment (start 177.899 108.899) (end 177.899 113.70204) (width 0.2) (layer "F.Cu") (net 3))
 (segment (start 166.0875 107) (end 167.4865 105.601) (width 0.2) (layer "F.Cu") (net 3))
 (segment (start 167.4865 105.601) (end 174.601 105.601) (width 0.2) (layer "F.Cu") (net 3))
 (segment (start 166.0875 107.25) (end 166.0875 107) (width 0.2) (layer "F.Cu") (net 3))
 (segment (start 177.60104 114) (end 177 114) (width 0.2) (layer "F.Cu") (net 3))
 (segment (start 176.7 114.3) (end 172.5 114.3) (width 0.2) (layer "F.Cu") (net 3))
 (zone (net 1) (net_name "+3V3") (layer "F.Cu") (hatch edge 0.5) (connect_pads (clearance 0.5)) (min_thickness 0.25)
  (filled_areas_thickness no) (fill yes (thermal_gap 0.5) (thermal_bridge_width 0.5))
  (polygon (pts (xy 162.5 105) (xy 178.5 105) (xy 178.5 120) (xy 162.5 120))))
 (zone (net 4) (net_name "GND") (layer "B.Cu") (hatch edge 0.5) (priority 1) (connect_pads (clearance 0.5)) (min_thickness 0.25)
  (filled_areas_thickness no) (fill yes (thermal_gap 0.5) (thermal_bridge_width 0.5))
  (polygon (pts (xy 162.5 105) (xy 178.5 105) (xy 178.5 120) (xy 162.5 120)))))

